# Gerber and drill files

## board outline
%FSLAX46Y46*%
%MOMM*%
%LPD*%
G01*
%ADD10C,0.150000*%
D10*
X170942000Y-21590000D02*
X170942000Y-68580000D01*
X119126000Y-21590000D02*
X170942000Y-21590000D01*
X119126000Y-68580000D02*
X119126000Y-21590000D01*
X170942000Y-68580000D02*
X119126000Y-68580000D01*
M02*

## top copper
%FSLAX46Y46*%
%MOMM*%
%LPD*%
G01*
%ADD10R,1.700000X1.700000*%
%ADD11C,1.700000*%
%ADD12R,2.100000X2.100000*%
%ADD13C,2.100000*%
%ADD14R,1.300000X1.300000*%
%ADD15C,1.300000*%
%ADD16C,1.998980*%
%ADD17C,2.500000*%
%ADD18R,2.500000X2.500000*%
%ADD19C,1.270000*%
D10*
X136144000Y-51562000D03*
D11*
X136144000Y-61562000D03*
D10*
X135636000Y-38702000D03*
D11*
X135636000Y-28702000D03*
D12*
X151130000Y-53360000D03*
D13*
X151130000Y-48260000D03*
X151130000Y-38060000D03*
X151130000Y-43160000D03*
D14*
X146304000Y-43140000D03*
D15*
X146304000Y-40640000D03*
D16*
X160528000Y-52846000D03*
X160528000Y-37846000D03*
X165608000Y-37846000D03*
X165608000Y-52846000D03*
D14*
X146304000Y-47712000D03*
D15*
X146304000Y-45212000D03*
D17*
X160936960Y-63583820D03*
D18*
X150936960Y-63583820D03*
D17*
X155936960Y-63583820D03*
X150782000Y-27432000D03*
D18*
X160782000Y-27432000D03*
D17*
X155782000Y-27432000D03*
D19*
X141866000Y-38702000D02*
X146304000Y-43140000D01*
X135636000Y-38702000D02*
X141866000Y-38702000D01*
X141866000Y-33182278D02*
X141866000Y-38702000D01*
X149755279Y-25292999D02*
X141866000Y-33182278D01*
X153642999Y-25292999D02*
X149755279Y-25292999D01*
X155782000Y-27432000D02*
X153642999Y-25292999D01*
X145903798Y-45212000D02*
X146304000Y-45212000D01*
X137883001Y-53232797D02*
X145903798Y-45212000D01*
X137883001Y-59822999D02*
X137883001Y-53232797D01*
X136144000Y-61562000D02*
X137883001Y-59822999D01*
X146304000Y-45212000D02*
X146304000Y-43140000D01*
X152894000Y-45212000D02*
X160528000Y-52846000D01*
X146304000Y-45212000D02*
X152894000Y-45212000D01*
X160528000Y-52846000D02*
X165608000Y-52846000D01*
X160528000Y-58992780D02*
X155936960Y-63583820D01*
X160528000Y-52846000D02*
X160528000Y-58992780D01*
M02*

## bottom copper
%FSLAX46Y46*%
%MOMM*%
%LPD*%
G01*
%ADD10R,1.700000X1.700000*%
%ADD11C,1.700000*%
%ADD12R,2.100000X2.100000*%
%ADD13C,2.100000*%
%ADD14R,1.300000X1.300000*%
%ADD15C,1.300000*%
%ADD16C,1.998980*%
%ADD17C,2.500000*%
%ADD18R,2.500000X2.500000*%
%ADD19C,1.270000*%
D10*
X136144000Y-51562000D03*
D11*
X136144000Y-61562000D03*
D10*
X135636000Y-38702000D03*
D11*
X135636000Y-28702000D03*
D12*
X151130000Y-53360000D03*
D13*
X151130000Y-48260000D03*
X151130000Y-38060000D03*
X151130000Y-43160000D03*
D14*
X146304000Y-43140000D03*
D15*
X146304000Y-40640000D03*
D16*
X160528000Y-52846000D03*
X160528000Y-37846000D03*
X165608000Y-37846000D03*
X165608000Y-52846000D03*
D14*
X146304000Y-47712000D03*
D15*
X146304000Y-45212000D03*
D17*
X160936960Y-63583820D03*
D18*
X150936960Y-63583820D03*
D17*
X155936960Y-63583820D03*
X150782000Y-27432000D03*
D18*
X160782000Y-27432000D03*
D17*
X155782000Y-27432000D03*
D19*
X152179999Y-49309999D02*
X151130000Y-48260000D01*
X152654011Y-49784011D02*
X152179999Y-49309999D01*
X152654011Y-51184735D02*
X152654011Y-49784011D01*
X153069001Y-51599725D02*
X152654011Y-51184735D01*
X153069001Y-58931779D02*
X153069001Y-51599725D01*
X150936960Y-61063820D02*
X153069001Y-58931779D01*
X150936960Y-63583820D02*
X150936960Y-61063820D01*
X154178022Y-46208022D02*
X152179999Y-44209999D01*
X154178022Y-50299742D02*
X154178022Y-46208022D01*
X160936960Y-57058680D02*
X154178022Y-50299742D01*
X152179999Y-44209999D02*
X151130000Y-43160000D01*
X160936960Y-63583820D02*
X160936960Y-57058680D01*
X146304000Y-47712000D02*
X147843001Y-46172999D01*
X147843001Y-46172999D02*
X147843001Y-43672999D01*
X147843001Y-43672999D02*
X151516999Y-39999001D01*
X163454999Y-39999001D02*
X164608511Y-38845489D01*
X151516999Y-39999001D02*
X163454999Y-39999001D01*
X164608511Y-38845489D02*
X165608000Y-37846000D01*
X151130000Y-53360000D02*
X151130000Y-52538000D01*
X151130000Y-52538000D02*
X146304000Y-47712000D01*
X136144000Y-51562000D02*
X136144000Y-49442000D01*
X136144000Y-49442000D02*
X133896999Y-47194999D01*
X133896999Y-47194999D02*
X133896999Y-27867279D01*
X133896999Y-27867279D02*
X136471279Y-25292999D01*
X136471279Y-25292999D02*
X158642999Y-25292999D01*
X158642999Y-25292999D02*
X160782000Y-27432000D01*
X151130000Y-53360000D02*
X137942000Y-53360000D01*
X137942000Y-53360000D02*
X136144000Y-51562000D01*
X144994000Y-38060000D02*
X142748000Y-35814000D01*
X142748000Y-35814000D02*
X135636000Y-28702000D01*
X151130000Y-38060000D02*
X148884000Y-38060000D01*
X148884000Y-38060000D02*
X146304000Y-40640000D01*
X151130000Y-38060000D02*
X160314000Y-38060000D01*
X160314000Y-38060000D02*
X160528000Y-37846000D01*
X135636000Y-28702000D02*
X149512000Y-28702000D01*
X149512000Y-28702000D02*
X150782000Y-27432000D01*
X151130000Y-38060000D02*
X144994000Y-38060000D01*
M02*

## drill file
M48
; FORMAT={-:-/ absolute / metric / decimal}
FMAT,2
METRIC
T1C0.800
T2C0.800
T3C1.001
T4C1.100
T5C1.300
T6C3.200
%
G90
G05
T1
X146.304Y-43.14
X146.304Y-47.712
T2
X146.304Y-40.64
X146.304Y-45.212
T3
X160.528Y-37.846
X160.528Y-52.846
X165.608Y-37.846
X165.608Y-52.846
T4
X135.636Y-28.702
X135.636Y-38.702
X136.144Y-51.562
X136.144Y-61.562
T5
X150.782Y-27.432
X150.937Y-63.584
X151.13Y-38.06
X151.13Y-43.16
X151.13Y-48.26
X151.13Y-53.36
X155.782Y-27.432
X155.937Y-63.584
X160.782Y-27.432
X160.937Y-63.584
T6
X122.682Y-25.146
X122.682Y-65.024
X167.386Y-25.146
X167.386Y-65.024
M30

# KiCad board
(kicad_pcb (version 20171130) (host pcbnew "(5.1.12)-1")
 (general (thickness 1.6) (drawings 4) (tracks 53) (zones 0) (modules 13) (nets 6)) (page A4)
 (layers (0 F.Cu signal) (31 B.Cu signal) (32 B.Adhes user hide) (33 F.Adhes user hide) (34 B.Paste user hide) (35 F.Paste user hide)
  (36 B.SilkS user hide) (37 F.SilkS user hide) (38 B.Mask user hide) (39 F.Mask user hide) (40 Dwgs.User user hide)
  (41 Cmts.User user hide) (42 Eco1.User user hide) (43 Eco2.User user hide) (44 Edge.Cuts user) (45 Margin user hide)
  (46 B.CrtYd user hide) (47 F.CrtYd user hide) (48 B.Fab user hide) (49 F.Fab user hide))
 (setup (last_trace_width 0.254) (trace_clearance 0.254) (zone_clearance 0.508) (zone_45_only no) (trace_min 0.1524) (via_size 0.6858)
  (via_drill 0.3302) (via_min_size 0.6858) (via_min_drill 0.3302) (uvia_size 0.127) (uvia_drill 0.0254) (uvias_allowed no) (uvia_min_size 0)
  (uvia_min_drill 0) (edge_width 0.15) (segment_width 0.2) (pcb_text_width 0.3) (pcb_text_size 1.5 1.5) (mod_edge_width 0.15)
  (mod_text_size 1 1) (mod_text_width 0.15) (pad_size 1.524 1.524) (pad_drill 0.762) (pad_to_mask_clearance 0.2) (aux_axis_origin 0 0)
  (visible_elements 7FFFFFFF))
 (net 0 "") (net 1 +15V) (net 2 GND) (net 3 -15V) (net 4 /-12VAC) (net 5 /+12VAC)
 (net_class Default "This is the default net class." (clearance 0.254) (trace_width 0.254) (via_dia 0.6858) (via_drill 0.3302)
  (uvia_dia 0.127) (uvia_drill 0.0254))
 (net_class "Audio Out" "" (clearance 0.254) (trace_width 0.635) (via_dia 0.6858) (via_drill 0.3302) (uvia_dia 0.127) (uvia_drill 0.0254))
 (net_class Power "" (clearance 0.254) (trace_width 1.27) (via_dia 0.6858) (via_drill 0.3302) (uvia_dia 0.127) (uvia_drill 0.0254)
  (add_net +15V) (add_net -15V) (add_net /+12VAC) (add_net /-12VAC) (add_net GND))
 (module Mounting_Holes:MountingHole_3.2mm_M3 (layer F.Cu) (at 122.682 25.146)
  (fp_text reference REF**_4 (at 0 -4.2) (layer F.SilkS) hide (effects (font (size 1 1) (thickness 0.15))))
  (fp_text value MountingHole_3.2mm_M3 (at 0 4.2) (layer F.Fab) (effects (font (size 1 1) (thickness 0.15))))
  (pad 1 np_thru_hole circle (at 0 0) (size 3.2 3.2) (drill 3.2) (layers *.Cu *.Mask)))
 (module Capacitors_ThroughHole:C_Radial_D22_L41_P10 (layer F.Cu) (at 136.144 51.562 270)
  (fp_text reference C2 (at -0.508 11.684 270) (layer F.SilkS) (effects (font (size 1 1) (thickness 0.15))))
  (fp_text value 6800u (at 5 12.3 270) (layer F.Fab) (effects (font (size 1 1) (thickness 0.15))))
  (pad 1 thru_hole rect (at 0 0 270) (size 1.7 1.7) (drill 1.1) (layers *.Cu *.Mask) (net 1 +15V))
  (pad 2 thru_hole circle (at 10 0 270) (size 1.7 1.7) (drill 1.1) (layers *.Cu *.Mask) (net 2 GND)))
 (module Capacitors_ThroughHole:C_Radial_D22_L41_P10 (layer F.Cu) (at 135.636 38.702 90)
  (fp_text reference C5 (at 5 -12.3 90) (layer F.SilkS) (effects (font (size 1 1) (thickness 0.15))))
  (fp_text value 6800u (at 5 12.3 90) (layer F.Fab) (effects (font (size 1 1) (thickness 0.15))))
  (pad 1 thru_hole rect (at 0 0 90) (size 1.7 1.7) (drill 1.1) (layers *.Cu *.Mask) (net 2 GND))
  (pad 2 thru_hole circle (at 10 0 90) (size 1.7 1.7) (drill 1.1) (layers *.Cu *.Mask) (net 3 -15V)))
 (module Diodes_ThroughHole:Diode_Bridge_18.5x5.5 (layer F.Cu) (at 151.13 53.36 90)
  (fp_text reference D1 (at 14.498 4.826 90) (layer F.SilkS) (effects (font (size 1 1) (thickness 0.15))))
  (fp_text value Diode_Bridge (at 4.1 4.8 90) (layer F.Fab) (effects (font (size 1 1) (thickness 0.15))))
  (pad 3 thru_hole rect (at 0 0 90) (size 2.1 2.1) (drill 1.3) (layers *.Cu *.Mask) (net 1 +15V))
  (pad 2 thru_hole circle (at 5.1 0 90) (size 2.1 2.1) (drill 1.3) (layers *.Cu *.Mask) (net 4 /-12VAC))
  (pad 1 thru_hole circle (at 15.3 0 90) (size 2.1 2.1) (drill 1.3) (layers *.Cu *.Mask) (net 3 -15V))
  (pad 4 thru_hole circle (at 10.2 0 90) (size 2.1 2.1) (drill 1.3) (layers *.Cu *.Mask) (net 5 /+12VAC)))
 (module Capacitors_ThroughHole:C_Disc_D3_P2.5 (layer F.Cu) (at 146.304 43.14 90)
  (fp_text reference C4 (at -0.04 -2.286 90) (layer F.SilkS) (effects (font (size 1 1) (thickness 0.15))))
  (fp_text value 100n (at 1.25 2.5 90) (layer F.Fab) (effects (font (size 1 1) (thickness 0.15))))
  (pad 1 thru_hole rect (at 0 0 90) (size 1.3 1.3) (drill 0.8) (layers *.Cu *.Mask) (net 2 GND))
  (pad 2 thru_hole circle (at 2.5 0 90) (size 1.3 1.3) (drill 0.8001) (layers *.Cu *.Mask) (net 3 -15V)))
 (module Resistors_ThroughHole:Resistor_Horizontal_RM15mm (layer F.Cu) (at 160.528 52.846 90)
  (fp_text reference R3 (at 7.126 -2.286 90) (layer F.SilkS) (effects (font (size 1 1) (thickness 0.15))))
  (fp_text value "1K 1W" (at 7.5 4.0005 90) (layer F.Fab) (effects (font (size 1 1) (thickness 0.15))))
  (pad 1 thru_hole circle (at 0 0 90) (size 1.99898 1.99898) (drill 1.00076) (layers *.Cu *.SilkS *.Mask) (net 2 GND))
  (pad 2 thru_hole circle (at 15 0 90) (size 1.99898 1.99898) (drill 1.00076) (layers *.Cu *.SilkS *.Mask) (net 3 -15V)))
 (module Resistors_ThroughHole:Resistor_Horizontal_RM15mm (layer F.Cu) (at 165.608 37.846 270)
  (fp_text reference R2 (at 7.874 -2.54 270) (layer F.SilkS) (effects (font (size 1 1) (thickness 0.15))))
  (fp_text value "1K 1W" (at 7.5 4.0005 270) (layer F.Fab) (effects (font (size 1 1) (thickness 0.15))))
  (pad 1 thru_hole circle (at 0 0 270) (size 1.99898 1.99898) (drill 1.00076) (layers *.Cu *.SilkS *.Mask) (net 1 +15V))
  (pad 2 thru_hole circle (at 15 0 270) (size 1.99898 1.99898) (drill 1.00076) (layers *.Cu *.SilkS *.Mask) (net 2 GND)))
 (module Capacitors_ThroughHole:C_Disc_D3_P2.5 (layer F.Cu) (at 146.304 47.712 90)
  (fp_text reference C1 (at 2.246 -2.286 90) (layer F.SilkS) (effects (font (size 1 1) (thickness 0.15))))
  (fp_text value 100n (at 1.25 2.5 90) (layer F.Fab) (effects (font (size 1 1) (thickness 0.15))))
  (pad 1 thru_hole rect (at 0 0 90) (size 1.3 1.3) (drill 0.8) (layers *.Cu *.Mask) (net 1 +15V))
  (pad 2 thru_hole circle (at 2.5 0 90) (size 1.3 1.3) (drill 0.8001) (layers *.Cu *.Mask) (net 2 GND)))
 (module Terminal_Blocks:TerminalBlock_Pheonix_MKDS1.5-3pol (layer F.Cu) (at 150.93696 63.58382)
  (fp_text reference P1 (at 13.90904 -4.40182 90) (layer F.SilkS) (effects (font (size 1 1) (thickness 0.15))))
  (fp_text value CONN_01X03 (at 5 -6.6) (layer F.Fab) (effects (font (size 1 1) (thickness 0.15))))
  (pad 3 thru_hole circle (at 10 0) (size 2.5 2.5) (drill 1.3) (layers *.Cu *.Mask) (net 5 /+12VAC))
  (pad 1 thru_hole rect (at 0 0) (size 2.5 2.5) (drill 1.3) (layers *.Cu *.Mask) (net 4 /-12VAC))
  (pad 2 thru_hole circle (at 5 0) (size 2.5 2.5) (drill 1.3) (layers *.Cu *.Mask) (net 2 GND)))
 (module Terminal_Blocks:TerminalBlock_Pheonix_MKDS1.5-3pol (layer F.Cu) (at 160.782 27.432 180)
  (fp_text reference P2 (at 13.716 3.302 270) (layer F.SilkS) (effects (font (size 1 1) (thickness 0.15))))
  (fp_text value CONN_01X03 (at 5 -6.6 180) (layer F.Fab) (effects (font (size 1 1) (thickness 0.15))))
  (pad 3 thru_hole circle (at 10 0 180) (size 2.5 2.5) (drill 1.3) (layers *.Cu *.Mask) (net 3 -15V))
  (pad 1 thru_hole rect (at 0 0 180) (size 2.5 2.5) (drill 1.3) (layers *.Cu *.Mask) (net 1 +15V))
  (pad 2 thru_hole circle (at 5 0 180) (size 2.5 2.5) (drill 1.3) (layers *.Cu *.Mask) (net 2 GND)))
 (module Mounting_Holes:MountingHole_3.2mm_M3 (layer F.Cu) (at 167.386 25.146)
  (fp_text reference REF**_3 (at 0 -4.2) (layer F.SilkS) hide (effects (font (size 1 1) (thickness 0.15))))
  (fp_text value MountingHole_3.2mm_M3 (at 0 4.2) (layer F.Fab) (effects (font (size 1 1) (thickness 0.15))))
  (pad 1 np_thru_hole circle (at 0 0) (size 3.2 3.2) (drill 3.2) (layers *.Cu *.Mask)))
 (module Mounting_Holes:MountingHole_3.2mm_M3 (layer F.Cu) (at 167.386 65.024)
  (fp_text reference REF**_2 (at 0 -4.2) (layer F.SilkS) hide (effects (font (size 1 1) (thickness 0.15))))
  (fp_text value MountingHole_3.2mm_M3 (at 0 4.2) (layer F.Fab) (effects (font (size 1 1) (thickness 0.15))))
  (pad 1 np_thru_hole circle (at 0 0) (size 3.2 3.2) (drill 3.2) (layers *.Cu *.Mask)))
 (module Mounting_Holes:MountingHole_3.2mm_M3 (layer F.Cu) (at 122.682 65.024)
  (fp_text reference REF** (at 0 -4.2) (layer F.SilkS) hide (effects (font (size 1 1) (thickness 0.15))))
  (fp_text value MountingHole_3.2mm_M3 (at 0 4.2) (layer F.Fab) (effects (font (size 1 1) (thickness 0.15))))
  (pad 1 np_thru_hole circle (at 0 0) (size 3.2 3.2) (drill 3.2) (layers *.Cu *.Mask)))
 (gr_line (start 170.942 21.59) (end 170.942 68.58) (layer Edge.Cuts) (width 0.15))
 (gr_line (start 119.126 21.59) (end 170.942 21.59) (layer Edge.Cuts) (width 0.15))
 (gr_line (start 119.126 68.58) (end 119.126 21.59) (layer Edge.Cuts) (width 0.15))
 (gr_line (start 170.942 68.58) (end 119.126 68.58) (layer Edge.Cuts) (width 0.15))
 (segment (start 152.179999 49.309999) (end 151.13 48.26) (width 1.27) (layer B.Cu) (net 4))
 (segment (start 152.654011 49.784011) (end 152.179999 49.309999) (width 1.27) (layer B.Cu) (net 4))
 (segment (start 152.654011 51.184735) (end 152.654011 49.784011) (width 1.27) (layer B.Cu) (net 4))
 (segment (start 153.069001 51.599725) (end 152.654011 51.184735) (width 1.27) (layer B.Cu) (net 4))
 (segment (start 153.069001 58.931779) (end 153.069001 51.599725) (width 1.27) (layer B.Cu) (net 4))
 (segment (start 150.93696 61.06382) (end 153.069001 58.931779) (width 1.27) (layer B.Cu) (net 4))
 (segment (start 150.93696 63.58382) (end 150.93696 61.06382) (width 1.27) (layer B.Cu) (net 4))
 (segment (start 154.178022 46.208022) (end 152.179999 44.209999) (width 1.27) (layer B.Cu) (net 5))
 (segment (start 154.178022 50.299742) (end 154.178022 46.208022) (width 1.27) (layer B.Cu) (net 5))
 (segment (start 160.93696 57.05868) (end 154.178022 50.299742) (width 1.27) (layer B.Cu) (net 5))
 (segment (start 152.179999 44.209999) (end 151.13 43.16) (width 1.27) (layer B.Cu) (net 5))
 (segment (start 160.93696 63.58382) (end 160.93696 57.05868) (width 1.27) (layer B.Cu) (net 5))
 (segment (start 146.304 47.712) (end 147.843001 46.172999) (width 1.27) (layer B.Cu) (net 1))
 (segment (start 147.843001 46.172999) (end 147.843001 43.672999) (width 1.27) (layer B.Cu) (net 1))
 (segment (start 147.843001 43.672999) (end 151.516999 39.999001) (width 1.27) (layer B.Cu) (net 1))
 (segment (start 163.454999 39.999001) (end 164.608511 38.845489) (width 1.27) (layer B.Cu) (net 1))
 (segment (start 151.516999 39.999001) (end 163.454999 39.999001) (width 1.27) (layer B.Cu) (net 1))
 (segment (start 164.608511 38.845489) (end 165.608 37.846) (width 1.27) (layer B.Cu) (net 1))
 (segment (start 151.13 53.36) (end 151.13 52.538) (width 1.27) (layer B.Cu) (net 1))
 (segment (start 151.13 52.538) (end 146.304 47.712) (width 1.27) (layer B.Cu) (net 1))
 (segment (start 136.144 51.562) (end 136.144 49.442) (width 1.27) (layer B.Cu) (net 1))
 (segment (start 136.144 49.442) (end 133.896999 47.194999) (width 1.27) (layer B.Cu) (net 1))
 (segment (start 133.896999 47.194999) (end 133.896999 27.867279) (width 1.27) (layer B.Cu) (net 1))
 (segment (start 133.896999 27.867279) (end 136.471279 25.292999) (width 1.27) (layer B.Cu) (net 1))
 (segment (start 136.471279 25.292999) (end 158.642999 25.292999) (width 1.27) (layer B.Cu) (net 1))
 (segment (start 158.642999 25.292999) (end 160.782 27.432) (width 1.27) (layer B.Cu) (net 1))
 (segment (start 151.13 53.36) (end 137.942 53.36) (width 1.27) (layer B.Cu) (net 1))
 (segment (start 137.942 53.36) (end 136.144 51.562) (width 1.27) (layer B.Cu) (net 1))
 (segment (start 144.994 38.06) (end 142.748 35.814) (width 1.27) (layer B.Cu) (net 3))
 (segment (start 142.748 35.814) (end 135.636 28.702) (width 1.27) (layer B.Cu) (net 3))
 (segment (start 151.13 38.06) (end 148.884 38.06) (width 1.27) (layer B.Cu) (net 3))
 (segment (start 148.884 38.06) (end 146.304 40.64) (width 1.27) (layer B.Cu) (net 3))
 (segment (start 151.13 38.06) (end 160.314 38.06) (width 1.27) (layer B.Cu) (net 3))
 (segment (start 160.314 38.06) (end 160.528 37.846) (width 1.27) (layer B.Cu) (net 3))
 (segment (start 135.636 28.702) (end 149.512 28.702) (width 1.27) (layer B.Cu) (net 3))
 (segment (start 149.512 28.702) (end 150.782 27.432) (width 1.27) (layer B.Cu) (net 3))
 (segment (start 151.13 38.06) (end 144.994 38.06) (width 1.27) (layer B.Cu) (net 3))
 (segment (start 141.866 38.702) (end 146.304 43.14) (width 1.27) (layer F.Cu) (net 2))
 (segment (start 135.636 38.702) (end 141.866 38.702) (width 1.27) (layer F.Cu) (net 2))
 (segment (start 141.866 33.182278) (end 141.866 38.702) (width 1.27) (layer F.Cu) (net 2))
 (segment (start 149.755279 25.292999) (end 141.866 33.182278) (width 1.27) (layer F.Cu) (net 2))
 (segment (start 153.642999 25.292999) (end 149.755279 25.292999) (width 1.27) (layer F.Cu) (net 2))
 (segment (start 155.782 27.432) (end 153.642999 25.292999) (width 1.27) (layer F.Cu) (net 2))
 (segment (start 145.903798 45.212) (end 146.304 45.212) (width 1.27) (layer F.Cu) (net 2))
 (segment (start 137.883001 53.232797) (end 145.903798 45.212) (width 1.27) (layer F.Cu) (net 2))
 (segment (start 137.883001 59.822999) (end 137.883001 53.232797) (width 1.27) (layer F.Cu) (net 2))
 (segment (start 136.144 61.562) (end 137.883001 59.822999) (width 1.27) (layer F.Cu) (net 2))
 (segment (start 146.304 45.212) (end 146.304 43.14) (width 1.27) (layer F.Cu) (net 2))
 (segment (start 152.894 45.212) (end 160.528 52.846) (width 1.27) (layer F.Cu) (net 2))
 (segment (start 146.304 45.212) (end 152.894 45.212) (width 1.27) (layer F.Cu) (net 2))
 (segment (start 160.528 52.846) (end 165.608 52.846) (width 1.27) (layer F.Cu) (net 2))
 (segment (start 160.528 58.99278) (end 155.93696 63.58382) (width 1.27) (layer F.Cu) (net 2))
 (segment (start 160.528 52.846) (end 160.528 58.99278) (width 1.27) (layer F.Cu) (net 2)))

